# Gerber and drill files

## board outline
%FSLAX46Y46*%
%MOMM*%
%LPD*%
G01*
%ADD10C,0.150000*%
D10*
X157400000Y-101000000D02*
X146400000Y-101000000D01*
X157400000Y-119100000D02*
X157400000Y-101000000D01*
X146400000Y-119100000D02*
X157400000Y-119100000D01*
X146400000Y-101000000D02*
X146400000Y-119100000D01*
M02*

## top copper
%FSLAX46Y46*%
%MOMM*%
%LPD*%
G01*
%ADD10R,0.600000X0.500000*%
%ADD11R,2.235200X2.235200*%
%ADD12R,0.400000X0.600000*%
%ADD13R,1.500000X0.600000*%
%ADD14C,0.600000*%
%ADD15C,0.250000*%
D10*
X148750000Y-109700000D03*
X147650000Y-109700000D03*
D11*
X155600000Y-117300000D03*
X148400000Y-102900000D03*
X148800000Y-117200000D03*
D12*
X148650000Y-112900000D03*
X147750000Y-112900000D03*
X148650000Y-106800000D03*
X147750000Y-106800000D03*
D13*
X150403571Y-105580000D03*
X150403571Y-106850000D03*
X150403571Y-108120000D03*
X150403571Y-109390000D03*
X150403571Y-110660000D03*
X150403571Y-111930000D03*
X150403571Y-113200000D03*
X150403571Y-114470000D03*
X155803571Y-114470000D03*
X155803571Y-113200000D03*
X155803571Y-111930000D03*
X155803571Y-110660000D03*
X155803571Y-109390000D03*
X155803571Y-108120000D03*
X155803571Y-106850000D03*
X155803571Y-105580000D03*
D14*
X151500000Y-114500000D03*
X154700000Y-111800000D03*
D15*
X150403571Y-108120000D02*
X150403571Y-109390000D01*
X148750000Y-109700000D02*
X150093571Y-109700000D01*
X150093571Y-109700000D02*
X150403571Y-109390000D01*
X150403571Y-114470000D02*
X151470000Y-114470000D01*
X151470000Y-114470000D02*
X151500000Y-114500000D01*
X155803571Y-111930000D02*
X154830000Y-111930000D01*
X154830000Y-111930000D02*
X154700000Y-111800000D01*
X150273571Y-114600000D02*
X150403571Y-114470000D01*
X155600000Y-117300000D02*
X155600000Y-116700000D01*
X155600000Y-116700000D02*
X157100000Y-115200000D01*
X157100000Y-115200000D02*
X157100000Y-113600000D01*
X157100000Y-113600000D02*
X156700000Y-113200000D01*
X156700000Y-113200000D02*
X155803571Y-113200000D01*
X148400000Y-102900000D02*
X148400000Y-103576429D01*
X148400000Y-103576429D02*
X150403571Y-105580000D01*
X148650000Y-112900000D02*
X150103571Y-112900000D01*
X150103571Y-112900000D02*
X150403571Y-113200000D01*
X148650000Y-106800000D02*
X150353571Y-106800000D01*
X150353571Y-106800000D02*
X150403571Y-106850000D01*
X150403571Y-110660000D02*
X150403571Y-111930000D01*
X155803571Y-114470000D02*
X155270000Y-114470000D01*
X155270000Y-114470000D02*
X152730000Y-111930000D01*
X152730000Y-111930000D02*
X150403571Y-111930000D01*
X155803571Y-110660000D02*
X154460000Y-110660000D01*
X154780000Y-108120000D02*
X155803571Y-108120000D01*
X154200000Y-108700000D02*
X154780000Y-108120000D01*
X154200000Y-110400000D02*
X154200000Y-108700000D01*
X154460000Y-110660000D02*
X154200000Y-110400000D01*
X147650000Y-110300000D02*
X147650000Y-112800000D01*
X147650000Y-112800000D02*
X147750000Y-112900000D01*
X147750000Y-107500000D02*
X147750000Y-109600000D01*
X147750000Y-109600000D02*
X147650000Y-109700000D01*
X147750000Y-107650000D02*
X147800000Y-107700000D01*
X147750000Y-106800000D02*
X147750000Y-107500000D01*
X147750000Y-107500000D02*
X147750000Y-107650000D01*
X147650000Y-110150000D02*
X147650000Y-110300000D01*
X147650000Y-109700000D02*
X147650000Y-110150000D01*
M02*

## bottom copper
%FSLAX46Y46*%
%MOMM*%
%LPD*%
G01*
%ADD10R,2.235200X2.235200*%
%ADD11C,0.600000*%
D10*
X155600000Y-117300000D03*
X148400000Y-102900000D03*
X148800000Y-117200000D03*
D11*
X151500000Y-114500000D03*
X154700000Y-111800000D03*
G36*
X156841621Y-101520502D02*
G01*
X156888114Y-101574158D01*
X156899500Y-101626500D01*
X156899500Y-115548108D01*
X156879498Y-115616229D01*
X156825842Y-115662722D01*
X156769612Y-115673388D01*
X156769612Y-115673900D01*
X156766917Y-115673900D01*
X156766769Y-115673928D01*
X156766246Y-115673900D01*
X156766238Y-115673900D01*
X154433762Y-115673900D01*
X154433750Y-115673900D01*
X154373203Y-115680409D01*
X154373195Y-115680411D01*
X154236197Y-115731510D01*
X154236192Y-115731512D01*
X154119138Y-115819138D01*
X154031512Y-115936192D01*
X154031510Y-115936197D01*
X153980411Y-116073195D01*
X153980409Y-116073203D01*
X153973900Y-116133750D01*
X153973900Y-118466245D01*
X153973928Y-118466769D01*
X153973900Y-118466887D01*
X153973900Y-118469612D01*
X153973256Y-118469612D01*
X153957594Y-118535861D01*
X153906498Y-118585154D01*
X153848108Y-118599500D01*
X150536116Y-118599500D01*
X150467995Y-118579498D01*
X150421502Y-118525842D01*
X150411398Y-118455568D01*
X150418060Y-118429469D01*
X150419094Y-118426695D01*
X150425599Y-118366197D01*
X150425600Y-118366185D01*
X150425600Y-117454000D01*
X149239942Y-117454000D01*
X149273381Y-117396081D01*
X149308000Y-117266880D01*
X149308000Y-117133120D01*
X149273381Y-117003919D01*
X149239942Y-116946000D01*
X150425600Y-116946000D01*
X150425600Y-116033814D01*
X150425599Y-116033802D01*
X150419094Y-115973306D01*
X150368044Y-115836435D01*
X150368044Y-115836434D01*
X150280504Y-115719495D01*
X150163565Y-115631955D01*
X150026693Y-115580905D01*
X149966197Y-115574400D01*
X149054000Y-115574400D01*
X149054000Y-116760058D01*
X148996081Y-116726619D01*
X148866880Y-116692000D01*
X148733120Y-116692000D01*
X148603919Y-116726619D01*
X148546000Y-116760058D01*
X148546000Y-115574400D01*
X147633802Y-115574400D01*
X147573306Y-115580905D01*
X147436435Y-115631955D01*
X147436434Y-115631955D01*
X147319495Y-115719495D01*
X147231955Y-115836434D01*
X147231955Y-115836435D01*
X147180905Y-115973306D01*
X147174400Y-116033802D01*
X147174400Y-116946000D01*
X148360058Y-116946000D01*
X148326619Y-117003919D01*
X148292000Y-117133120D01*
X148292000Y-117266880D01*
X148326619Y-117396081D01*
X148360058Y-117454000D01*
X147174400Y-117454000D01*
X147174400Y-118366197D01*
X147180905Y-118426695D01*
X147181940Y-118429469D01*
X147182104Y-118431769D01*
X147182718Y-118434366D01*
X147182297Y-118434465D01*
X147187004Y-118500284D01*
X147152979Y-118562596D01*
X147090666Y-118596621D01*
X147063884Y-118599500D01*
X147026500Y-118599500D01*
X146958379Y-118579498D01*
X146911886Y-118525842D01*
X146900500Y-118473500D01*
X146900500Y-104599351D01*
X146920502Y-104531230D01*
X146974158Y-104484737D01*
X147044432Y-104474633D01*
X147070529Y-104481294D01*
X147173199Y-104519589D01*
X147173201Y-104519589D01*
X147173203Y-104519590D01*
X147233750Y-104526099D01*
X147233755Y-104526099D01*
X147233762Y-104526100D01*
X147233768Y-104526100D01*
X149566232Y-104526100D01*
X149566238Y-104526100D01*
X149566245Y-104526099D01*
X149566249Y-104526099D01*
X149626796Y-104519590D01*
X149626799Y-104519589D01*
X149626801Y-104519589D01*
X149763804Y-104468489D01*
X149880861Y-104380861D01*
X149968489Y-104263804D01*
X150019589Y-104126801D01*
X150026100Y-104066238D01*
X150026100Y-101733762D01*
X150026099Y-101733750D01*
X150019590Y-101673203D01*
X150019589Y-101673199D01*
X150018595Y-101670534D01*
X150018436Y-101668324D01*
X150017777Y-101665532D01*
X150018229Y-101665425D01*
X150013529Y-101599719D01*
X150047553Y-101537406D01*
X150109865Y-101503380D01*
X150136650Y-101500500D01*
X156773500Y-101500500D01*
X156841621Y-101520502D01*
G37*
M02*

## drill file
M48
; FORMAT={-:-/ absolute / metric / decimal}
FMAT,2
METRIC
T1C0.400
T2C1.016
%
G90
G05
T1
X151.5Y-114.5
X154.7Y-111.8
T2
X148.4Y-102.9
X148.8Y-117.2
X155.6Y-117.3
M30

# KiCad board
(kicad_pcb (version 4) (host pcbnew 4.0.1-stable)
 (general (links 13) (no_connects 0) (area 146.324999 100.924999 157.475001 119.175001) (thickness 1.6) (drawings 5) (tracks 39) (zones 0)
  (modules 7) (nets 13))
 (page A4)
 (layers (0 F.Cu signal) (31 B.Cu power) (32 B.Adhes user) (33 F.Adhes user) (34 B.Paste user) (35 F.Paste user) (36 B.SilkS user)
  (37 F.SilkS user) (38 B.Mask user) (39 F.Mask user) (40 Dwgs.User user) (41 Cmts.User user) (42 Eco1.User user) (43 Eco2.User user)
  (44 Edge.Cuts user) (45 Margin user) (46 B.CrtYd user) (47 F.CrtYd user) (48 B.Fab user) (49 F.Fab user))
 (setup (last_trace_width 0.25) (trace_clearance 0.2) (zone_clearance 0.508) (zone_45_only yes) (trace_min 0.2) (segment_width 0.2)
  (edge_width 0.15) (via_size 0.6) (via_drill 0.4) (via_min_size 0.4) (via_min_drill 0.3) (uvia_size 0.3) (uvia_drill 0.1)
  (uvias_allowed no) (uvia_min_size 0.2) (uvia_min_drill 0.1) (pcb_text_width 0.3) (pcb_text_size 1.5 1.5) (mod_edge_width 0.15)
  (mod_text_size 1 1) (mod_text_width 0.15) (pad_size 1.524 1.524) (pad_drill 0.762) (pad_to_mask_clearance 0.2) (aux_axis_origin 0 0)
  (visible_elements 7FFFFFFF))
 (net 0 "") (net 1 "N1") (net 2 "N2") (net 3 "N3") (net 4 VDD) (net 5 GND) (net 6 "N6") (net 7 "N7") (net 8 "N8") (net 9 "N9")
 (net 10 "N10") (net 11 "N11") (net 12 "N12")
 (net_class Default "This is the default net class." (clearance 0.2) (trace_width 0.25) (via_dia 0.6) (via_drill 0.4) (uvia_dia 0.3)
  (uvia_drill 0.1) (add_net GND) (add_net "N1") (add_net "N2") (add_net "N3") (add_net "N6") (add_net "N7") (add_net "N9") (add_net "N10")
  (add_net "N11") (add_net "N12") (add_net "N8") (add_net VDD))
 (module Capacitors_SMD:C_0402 (layer F.Cu) (at 148.2 109.7 180)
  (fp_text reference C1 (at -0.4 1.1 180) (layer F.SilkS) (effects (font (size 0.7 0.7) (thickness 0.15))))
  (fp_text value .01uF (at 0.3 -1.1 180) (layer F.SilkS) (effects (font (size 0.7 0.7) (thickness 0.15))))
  (pad 1 smd rect (at -0.55 0 180) (size 0.6 0.5) (layers F.Cu F.Paste F.Mask) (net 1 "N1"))
  (pad 2 smd rect (at 0.55 0 180) (size 0.6 0.5) (layers F.Cu F.Paste F.Mask) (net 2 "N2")))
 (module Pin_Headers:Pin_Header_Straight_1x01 (layer F.Cu) (at 155.6 117.3)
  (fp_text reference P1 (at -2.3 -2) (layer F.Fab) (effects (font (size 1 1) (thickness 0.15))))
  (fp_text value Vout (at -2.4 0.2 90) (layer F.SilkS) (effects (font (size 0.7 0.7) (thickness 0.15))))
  (pad 1 thru_hole rect (at 0 0) (size 2.2352 2.2352) (drill 1.016) (layers *.Cu *.Mask F.SilkS) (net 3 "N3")))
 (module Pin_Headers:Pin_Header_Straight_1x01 (layer F.Cu) (at 148.4 102.9)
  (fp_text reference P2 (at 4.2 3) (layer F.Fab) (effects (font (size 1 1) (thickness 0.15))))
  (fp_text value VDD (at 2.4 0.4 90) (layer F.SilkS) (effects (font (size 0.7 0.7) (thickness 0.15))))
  (pad 1 thru_hole rect (at 0 0) (size 2.2352 2.2352) (drill 1.016) (layers *.Cu *.Mask F.SilkS) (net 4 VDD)))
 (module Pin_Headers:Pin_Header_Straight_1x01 (layer F.Cu) (at 148.8 117.2)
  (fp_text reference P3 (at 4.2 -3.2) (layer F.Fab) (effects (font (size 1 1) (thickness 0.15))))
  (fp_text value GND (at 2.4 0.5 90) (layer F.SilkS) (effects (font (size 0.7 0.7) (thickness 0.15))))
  (pad 1 thru_hole rect (at 0 0) (size 2.2352 2.2352) (drill 1.016) (layers *.Cu *.Mask F.SilkS) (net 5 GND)))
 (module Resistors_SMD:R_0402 (layer F.Cu) (at 148.2 112.9 180)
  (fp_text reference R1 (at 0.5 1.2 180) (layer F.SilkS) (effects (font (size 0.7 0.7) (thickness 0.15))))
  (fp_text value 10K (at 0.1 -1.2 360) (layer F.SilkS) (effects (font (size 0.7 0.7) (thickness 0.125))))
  (pad 1 smd rect (at -0.45 0 180) (size 0.4 0.6) (layers F.Cu F.Paste F.Mask) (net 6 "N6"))
  (pad 2 smd rect (at 0.45 0 180) (size 0.4 0.6) (layers F.Cu F.Paste F.Mask) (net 2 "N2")))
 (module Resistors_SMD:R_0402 (layer F.Cu) (at 148.2 106.8 180)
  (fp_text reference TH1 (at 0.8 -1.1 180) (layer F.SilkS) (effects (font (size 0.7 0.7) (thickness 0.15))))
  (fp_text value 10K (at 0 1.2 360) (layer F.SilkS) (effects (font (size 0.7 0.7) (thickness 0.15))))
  (pad 1 smd rect (at -0.45 0 180) (size 0.4 0.6) (layers F.Cu F.Paste F.Mask) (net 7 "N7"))
  (pad 2 smd rect (at 0.45 0 180) (size 0.4 0.6) (layers F.Cu F.Paste F.Mask) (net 2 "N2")))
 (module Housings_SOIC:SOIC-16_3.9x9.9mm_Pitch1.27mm (layer F.Cu) (at 153.103571 110.025)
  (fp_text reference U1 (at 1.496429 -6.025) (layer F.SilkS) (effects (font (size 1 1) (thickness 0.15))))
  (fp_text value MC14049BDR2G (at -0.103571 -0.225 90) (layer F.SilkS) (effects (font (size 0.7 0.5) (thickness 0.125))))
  (pad 1 smd rect (at -2.7 -4.445) (size 1.5 0.6) (layers F.Cu F.Paste F.Mask) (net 4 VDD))
  (pad 2 smd rect (at -2.7 -3.175) (size 1.5 0.6) (layers F.Cu F.Paste F.Mask) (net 7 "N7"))
  (pad 3 smd rect (at -2.7 -1.905) (size 1.5 0.6) (layers F.Cu F.Paste F.Mask) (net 1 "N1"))
  (pad 4 smd rect (at -2.7 -0.635) (size 1.5 0.6) (layers F.Cu F.Paste F.Mask) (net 1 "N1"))
  (pad 5 smd rect (at -2.7 0.635) (size 1.5 0.6) (layers F.Cu F.Paste F.Mask) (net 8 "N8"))
  (pad 6 smd rect (at -2.7 1.905) (size 1.5 0.6) (layers F.Cu F.Paste F.Mask) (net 8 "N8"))
  (pad 7 smd rect (at -2.7 3.175) (size 1.5 0.6) (layers F.Cu F.Paste F.Mask) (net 6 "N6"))
  (pad 8 smd rect (at -2.7 4.445) (size 1.5 0.6) (layers F.Cu F.Paste F.Mask) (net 5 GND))
  (pad 9 smd rect (at 2.7 4.445) (size 1.5 0.6) (layers F.Cu F.Paste F.Mask) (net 8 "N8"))
  (pad 10 smd rect (at 2.7 3.175) (size 1.5 0.6) (layers F.Cu F.Paste F.Mask) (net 3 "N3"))
  (pad 11 smd rect (at 2.7 1.905) (size 1.5 0.6) (layers F.Cu F.Paste F.Mask) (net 5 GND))
  (pad 12 smd rect (at 2.7 0.635) (size 1.5 0.6) (layers F.Cu F.Paste F.Mask) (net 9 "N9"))
  (pad 13 smd rect (at 2.7 -0.635) (size 1.5 0.6) (layers F.Cu F.Paste F.Mask) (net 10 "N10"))
  (pad 14 smd rect (at 2.7 -1.905) (size 1.5 0.6) (layers F.Cu F.Paste F.Mask) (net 9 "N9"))
  (pad 15 smd rect (at 2.7 -3.175) (size 1.5 0.6) (layers F.Cu F.Paste F.Mask) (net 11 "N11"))
  (pad 16 smd rect (at 2.7 -4.445) (size 1.5 0.6) (layers F.Cu F.Paste F.Mask) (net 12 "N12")))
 (gr_line (start 157.4 101) (end 146.4 101) (angle 90) (layer Edge.Cuts) (width 0.15))
 (gr_line (start 157.4 119.1) (end 157.4 101) (angle 90) (layer Edge.Cuts) (width 0.15))
 (gr_line (start 146.4 119.1) (end 157.4 119.1) (angle 90) (layer Edge.Cuts) (width 0.15))
 (gr_line (start 146.4 101) (end 146.4 119.1) (angle 90) (layer Edge.Cuts) (width 0.15))
 (segment (start 150.403571 108.12) (end 150.403571 109.39) (width 0.25) (layer F.Cu) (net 1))
 (segment (start 148.75 109.7) (end 150.093571 109.7) (width 0.25) (layer F.Cu) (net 1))
 (segment (start 150.093571 109.7) (end 150.403571 109.39) (width 0.25) (layer F.Cu) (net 1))
 (segment (start 150.403571 114.47) (end 151.47 114.47) (width 0.25) (layer F.Cu) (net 5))
 (via (at 151.5 114.5) (size 0.6) (drill 0.4) (layers F.Cu B.Cu) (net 5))
 (segment (start 151.47 114.47) (end 151.5 114.5) (width 0.25) (layer F.Cu) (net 5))
 (segment (start 155.803571 111.93) (end 154.83 111.93) (width 0.25) (layer F.Cu) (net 5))
 (via (at 154.7 111.8) (size 0.6) (drill 0.4) (layers F.Cu B.Cu) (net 5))
 (segment (start 154.83 111.93) (end 154.7 111.8) (width 0.25) (layer F.Cu) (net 5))
 (segment (start 150.273571 114.6) (end 150.403571 114.47) (width 0.25) (layer F.Cu) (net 5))
 (segment (start 155.6 117.3) (end 155.6 116.7) (width 0.25) (layer F.Cu) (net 3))
 (segment (start 155.6 116.7) (end 157.1 115.2) (width 0.25) (layer F.Cu) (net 3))
 (segment (start 157.1 115.2) (end 157.1 113.6) (width 0.25) (layer F.Cu) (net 3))
 (segment (start 157.1 113.6) (end 156.7 113.2) (width 0.25) (layer F.Cu) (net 3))
 (segment (start 156.7 113.2) (end 155.803571 113.2) (width 0.25) (layer F.Cu) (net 3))
 (segment (start 148.4 102.9) (end 148.4 103.576429) (width 0.25) (layer F.Cu) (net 4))
 (segment (start 148.4 103.576429) (end 150.403571 105.58) (width 0.25) (layer F.Cu) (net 4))
 (segment (start 148.65 112.9) (end 150.103571 112.9) (width 0.25) (layer F.Cu) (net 6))
 (segment (start 150.103571 112.9) (end 150.403571 113.2) (width 0.25) (layer F.Cu) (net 6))
 (segment (start 148.65 106.8) (end 150.353571 106.8) (width 0.25) (layer F.Cu) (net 7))
 (segment (start 150.353571 106.8) (end 150.403571 106.85) (width 0.25) (layer F.Cu) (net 7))
 (segment (start 150.403571 110.66) (end 150.403571 111.93) (width 0.25) (layer F.Cu) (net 8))
 (segment (start 155.803571 114.47) (end 155.27 114.47) (width 0.25) (layer F.Cu) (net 8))
 (segment (start 155.27 114.47) (end 152.73 111.93) (width 0.25) (layer F.Cu) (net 8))
 (segment (start 152.73 111.93) (end 150.403571 111.93) (width 0.25) (layer F.Cu) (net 8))
 (segment (start 155.803571 110.66) (end 154.46 110.66) (width 0.25) (layer F.Cu) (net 9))
 (segment (start 154.78 108.12) (end 155.803571 108.12) (width 0.25) (layer F.Cu) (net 9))
 (segment (start 154.2 108.7) (end 154.78 108.12) (width 0.25) (layer F.Cu) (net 9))
 (segment (start 154.2 110.4) (end 154.2 108.7) (width 0.25) (layer F.Cu) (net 9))
 (segment (start 154.46 110.66) (end 154.2 110.4) (width 0.25) (layer F.Cu) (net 9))
 (segment (start 147.65 110.3) (end 147.65 112.8) (width 0.25) (layer F.Cu) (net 2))
 (segment (start 147.65 112.8) (end 147.75 112.9) (width 0.25) (layer F.Cu) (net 2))
 (segment (start 147.75 107.5) (end 147.75 109.6) (width 0.25) (layer F.Cu) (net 2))
 (segment (start 147.75 109.6) (end 147.65 109.7) (width 0.25) (layer F.Cu) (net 2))
 (segment (start 147.75 107.65) (end 147.8 107.7) (width 0.25) (layer F.Cu) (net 2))
 (segment (start 147.75 106.8) (end 147.75 107.5) (width 0.25) (layer F.Cu) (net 2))
 (segment (start 147.75 107.5) (end 147.75 107.65) (width 0.25) (layer F.Cu) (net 2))
 (segment (start 147.65 110.15) (end 147.65 110.3) (width 0.25) (layer F.Cu) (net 2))
 (segment (start 147.65 109.7) (end 147.65 110.15) (width 0.25) (layer F.Cu) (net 2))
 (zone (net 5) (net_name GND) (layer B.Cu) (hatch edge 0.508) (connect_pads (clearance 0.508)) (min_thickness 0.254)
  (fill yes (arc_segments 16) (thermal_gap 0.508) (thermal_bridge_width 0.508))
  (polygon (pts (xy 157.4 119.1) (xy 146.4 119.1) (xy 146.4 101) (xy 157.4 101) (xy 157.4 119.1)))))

